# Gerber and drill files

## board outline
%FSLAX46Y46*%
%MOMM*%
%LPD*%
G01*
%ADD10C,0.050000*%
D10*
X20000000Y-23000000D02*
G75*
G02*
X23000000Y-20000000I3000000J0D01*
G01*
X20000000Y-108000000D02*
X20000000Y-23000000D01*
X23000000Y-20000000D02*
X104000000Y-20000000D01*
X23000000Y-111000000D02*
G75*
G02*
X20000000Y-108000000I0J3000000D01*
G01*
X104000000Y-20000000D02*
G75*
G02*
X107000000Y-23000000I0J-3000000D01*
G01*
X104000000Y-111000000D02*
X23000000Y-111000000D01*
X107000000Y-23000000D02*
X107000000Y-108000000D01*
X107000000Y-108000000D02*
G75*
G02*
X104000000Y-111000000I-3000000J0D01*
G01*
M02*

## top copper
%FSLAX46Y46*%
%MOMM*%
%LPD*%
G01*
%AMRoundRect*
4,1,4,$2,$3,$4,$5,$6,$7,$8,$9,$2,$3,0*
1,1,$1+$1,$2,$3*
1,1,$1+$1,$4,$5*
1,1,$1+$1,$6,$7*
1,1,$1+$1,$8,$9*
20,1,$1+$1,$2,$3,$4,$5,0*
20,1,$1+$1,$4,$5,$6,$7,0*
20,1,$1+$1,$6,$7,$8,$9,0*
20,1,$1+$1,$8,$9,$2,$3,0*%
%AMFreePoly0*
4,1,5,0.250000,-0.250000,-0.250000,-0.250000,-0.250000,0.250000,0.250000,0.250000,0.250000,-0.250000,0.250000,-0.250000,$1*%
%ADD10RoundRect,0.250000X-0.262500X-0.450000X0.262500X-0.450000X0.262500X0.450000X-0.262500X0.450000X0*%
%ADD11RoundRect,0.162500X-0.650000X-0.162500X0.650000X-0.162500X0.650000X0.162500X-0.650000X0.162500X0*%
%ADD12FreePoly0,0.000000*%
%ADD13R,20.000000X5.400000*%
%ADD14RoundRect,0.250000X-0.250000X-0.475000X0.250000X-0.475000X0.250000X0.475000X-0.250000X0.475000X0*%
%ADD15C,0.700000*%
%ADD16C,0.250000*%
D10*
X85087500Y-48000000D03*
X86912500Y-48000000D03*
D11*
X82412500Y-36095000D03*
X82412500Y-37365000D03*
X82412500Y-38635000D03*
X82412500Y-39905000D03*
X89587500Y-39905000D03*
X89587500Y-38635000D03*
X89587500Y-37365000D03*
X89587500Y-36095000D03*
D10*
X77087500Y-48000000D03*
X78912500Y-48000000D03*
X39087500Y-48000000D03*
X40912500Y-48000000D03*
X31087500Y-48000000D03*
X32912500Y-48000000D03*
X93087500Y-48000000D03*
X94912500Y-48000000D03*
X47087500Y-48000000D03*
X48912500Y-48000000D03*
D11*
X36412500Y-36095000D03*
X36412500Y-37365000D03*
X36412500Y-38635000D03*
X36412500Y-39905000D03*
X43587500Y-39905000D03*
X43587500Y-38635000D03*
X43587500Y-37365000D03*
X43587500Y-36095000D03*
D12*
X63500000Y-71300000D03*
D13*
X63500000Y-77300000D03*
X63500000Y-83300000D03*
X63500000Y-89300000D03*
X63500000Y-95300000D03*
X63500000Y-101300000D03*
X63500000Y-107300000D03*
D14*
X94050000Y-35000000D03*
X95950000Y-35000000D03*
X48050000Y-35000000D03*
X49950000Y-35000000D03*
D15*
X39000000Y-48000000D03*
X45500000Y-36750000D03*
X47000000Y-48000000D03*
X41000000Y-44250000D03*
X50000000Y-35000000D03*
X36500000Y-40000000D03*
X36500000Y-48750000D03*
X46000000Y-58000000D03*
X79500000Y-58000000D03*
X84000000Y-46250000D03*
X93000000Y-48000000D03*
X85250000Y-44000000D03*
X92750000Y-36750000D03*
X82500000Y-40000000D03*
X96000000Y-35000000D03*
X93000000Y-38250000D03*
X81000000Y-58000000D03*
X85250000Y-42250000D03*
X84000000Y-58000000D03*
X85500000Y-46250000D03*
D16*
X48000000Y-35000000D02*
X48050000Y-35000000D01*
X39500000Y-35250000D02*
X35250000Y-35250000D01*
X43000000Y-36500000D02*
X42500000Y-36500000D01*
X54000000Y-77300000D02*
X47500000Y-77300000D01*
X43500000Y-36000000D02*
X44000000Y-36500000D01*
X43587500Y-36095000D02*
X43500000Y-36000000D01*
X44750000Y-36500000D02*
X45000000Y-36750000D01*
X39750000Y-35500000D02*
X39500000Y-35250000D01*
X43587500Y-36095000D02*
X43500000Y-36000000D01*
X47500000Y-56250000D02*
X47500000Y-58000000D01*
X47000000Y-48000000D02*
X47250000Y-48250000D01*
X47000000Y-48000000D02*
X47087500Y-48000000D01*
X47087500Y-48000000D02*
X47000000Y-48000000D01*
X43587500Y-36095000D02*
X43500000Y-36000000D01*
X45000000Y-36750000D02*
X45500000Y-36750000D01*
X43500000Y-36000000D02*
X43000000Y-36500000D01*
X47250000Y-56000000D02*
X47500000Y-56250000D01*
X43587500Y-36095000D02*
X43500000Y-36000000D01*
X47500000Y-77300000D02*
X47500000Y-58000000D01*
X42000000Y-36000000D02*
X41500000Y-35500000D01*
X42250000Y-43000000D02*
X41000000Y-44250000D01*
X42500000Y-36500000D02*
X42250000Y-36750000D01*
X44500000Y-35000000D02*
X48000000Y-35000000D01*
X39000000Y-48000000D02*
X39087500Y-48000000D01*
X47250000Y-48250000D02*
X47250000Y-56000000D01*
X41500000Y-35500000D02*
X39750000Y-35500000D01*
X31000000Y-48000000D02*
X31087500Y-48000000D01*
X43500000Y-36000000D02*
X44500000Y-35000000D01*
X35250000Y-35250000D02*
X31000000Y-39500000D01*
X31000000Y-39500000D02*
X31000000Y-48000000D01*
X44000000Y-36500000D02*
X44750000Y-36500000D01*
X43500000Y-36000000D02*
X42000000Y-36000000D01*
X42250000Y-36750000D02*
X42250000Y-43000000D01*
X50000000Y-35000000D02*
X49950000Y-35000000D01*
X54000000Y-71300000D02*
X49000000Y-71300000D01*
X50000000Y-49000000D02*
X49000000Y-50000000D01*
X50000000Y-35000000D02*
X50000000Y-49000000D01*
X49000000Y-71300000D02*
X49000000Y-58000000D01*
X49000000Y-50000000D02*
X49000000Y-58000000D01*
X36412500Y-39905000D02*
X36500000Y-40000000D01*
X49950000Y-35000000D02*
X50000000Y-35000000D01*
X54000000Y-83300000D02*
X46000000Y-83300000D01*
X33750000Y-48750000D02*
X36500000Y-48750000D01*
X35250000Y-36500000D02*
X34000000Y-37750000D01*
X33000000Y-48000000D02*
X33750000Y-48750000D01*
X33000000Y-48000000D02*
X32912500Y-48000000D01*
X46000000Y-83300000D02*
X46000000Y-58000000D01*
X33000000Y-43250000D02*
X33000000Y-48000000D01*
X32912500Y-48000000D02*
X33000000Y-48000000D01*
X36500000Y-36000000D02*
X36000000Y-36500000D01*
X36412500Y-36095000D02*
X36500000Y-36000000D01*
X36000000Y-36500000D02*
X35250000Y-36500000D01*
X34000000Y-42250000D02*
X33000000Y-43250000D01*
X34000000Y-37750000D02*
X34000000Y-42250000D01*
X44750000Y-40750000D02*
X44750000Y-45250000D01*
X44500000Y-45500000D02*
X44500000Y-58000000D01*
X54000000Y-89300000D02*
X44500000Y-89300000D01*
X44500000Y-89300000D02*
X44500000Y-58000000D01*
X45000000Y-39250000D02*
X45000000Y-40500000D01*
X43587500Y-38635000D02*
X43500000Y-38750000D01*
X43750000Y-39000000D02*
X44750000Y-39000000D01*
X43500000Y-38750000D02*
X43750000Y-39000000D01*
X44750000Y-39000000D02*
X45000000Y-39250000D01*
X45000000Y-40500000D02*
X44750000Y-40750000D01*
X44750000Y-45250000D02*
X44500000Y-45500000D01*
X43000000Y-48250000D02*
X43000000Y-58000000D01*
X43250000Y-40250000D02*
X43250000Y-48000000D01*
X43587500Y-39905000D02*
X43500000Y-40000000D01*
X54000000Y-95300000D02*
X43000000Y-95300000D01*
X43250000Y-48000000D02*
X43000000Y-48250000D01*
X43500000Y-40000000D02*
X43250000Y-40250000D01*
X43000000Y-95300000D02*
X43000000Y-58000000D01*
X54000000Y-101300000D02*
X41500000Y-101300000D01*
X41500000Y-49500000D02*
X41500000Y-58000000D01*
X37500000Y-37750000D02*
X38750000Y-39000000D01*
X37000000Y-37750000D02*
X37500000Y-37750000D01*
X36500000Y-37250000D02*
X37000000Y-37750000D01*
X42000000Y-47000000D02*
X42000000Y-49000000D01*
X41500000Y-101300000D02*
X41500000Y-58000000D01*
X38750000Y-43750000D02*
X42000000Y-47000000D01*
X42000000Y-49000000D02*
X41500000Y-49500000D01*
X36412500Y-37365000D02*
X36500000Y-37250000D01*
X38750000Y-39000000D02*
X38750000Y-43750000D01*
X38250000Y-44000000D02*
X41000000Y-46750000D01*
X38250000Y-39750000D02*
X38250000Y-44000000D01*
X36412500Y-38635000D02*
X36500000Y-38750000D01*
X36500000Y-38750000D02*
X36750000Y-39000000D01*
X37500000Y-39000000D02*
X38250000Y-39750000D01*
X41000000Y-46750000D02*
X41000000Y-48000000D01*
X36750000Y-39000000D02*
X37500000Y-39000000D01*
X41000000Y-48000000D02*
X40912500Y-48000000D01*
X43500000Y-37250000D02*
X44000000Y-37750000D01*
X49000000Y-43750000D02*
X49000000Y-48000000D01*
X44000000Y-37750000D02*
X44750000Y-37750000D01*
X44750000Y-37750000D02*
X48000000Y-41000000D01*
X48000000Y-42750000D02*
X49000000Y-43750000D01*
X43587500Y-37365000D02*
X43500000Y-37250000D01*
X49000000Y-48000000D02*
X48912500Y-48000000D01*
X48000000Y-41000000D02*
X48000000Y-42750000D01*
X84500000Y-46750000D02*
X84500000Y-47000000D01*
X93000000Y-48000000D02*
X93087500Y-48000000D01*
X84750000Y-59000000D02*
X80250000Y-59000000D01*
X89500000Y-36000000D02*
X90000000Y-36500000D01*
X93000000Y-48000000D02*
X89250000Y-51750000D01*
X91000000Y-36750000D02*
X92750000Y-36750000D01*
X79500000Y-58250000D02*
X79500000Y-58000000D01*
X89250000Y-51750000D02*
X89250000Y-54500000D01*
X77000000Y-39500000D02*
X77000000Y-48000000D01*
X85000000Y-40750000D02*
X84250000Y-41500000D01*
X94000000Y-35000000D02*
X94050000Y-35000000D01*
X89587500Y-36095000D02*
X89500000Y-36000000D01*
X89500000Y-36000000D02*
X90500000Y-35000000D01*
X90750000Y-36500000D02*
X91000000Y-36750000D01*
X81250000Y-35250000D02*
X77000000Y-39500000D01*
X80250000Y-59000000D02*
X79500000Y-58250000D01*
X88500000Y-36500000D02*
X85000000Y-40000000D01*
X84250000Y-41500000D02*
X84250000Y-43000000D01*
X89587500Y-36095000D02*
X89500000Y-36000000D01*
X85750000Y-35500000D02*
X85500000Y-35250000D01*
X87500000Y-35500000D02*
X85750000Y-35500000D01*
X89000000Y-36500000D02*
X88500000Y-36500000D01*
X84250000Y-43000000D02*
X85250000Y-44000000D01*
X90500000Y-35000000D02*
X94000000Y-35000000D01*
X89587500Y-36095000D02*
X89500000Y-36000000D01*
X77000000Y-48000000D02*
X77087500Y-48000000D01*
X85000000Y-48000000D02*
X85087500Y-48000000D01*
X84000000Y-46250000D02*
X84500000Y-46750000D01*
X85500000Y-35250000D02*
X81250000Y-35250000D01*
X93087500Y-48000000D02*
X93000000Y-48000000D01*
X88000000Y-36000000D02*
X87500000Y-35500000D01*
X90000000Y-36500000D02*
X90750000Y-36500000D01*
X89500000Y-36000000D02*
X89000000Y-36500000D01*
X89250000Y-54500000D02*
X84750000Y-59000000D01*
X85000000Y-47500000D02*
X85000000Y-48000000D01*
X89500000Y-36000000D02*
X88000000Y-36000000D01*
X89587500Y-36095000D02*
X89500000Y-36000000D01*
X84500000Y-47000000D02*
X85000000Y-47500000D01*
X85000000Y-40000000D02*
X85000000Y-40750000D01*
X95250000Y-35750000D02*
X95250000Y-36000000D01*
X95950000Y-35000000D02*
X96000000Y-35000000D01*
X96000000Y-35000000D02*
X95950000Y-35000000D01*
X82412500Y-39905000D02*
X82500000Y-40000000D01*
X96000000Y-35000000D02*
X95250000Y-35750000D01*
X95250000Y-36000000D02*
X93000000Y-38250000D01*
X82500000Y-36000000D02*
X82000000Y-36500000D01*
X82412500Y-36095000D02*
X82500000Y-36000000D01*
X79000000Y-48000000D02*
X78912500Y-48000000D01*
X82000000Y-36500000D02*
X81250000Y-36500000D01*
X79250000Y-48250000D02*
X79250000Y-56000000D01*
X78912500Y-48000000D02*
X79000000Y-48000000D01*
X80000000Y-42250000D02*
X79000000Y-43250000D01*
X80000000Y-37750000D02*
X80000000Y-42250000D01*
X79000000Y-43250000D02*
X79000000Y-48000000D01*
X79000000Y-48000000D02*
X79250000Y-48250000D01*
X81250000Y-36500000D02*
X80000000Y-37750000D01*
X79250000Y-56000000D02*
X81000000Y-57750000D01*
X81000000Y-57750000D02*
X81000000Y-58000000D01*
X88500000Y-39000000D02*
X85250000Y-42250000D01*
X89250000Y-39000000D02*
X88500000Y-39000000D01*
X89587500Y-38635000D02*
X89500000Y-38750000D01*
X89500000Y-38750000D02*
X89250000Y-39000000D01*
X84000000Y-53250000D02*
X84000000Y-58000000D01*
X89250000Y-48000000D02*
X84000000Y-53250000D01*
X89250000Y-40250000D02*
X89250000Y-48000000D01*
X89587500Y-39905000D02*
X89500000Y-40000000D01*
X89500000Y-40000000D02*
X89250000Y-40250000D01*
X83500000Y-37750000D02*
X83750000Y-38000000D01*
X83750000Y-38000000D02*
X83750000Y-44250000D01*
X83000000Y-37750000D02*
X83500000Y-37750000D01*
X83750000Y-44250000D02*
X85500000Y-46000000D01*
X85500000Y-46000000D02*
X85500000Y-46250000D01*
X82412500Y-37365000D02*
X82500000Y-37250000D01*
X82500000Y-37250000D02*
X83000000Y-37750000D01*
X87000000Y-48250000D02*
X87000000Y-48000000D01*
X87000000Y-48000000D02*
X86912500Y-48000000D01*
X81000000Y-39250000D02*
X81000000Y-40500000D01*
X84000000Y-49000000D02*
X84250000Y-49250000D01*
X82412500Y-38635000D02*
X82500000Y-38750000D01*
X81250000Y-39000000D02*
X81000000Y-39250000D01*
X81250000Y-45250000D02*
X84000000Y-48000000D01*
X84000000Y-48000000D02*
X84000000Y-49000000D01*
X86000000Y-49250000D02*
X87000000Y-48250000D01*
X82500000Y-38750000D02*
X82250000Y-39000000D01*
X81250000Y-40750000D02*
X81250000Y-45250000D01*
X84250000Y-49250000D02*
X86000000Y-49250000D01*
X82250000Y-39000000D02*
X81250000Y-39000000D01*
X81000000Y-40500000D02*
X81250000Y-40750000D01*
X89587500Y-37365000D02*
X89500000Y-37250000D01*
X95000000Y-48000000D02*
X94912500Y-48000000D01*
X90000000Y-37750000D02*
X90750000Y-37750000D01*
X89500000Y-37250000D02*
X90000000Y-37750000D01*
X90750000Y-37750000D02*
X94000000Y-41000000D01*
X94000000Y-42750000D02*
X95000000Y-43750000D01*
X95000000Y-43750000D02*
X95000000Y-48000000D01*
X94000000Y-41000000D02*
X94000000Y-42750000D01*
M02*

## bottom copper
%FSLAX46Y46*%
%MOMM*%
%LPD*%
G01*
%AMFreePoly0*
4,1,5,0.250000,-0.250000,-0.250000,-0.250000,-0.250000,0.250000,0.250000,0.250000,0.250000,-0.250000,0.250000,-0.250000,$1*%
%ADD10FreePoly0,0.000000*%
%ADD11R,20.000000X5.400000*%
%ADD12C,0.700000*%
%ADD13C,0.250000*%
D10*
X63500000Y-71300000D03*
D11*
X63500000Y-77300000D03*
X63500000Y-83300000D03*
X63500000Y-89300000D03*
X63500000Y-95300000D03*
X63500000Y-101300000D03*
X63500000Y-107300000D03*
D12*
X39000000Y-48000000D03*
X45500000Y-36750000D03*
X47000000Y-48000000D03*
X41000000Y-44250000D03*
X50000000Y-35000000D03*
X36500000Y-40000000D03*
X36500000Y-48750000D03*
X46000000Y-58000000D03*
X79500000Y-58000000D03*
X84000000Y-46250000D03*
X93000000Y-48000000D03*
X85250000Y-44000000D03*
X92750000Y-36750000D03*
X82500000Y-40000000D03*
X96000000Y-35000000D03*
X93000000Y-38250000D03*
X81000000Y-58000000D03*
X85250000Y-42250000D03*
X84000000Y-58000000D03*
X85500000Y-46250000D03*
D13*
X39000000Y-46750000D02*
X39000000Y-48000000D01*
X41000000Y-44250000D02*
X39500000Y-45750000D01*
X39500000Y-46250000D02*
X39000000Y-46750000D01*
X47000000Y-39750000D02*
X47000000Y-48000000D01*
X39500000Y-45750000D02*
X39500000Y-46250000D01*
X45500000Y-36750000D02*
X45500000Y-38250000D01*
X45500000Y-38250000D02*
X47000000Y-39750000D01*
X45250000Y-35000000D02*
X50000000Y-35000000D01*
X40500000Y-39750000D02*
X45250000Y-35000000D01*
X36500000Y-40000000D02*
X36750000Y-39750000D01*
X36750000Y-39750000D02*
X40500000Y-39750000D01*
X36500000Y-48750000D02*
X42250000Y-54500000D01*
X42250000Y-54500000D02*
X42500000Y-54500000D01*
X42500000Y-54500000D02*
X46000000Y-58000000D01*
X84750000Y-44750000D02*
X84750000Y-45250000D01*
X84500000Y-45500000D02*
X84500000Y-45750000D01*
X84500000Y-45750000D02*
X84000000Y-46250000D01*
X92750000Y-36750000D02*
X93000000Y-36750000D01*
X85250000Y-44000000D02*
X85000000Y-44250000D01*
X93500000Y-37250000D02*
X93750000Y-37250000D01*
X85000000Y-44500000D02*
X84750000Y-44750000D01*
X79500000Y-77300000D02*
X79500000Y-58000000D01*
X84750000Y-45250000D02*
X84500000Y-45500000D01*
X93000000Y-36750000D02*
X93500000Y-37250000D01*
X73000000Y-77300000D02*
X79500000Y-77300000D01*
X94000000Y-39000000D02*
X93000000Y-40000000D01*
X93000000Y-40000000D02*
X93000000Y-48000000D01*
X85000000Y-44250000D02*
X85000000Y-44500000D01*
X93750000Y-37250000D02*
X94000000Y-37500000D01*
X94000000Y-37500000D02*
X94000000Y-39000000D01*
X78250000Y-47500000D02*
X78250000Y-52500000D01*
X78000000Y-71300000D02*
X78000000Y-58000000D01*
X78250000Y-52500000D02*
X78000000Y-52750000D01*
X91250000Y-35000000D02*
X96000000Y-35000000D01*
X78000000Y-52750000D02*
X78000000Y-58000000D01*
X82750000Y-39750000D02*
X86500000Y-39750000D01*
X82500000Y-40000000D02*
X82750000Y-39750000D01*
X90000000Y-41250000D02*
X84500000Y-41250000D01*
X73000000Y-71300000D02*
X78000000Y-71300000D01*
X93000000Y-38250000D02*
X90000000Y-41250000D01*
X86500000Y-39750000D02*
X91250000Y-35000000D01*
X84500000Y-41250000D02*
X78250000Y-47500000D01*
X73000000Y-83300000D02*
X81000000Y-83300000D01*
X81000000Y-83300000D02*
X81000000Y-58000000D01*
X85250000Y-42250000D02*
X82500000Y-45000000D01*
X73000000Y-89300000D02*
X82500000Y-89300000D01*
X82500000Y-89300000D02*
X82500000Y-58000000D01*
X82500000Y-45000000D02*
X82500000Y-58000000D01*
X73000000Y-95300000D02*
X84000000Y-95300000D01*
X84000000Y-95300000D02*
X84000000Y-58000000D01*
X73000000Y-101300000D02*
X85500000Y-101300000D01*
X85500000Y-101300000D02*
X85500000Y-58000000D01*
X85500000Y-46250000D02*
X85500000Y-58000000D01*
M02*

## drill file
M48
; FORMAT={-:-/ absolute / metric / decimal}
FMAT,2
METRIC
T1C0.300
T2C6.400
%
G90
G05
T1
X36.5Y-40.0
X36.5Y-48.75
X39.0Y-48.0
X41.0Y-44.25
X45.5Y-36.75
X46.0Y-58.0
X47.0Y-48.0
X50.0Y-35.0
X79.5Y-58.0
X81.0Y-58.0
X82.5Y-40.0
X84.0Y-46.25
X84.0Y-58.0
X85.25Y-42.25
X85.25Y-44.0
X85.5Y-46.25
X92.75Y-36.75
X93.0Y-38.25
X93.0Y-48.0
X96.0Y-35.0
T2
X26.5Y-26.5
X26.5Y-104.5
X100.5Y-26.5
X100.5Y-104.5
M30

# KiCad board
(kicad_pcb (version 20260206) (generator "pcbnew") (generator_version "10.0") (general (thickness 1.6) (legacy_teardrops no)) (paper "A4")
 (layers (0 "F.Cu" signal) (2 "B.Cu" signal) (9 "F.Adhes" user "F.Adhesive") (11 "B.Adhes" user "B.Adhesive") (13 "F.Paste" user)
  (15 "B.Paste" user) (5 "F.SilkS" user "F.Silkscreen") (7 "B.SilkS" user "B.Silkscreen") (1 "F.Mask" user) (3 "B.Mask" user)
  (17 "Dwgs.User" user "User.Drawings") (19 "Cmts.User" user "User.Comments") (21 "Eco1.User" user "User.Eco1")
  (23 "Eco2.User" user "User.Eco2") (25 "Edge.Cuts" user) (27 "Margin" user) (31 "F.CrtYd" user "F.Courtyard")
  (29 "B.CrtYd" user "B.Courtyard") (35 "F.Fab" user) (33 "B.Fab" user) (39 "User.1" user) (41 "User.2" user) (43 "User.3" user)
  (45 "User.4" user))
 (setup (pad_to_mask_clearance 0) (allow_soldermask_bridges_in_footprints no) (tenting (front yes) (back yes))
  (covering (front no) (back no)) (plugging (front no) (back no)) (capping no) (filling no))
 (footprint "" (layer "F.Cu") (at 100.5 104.5)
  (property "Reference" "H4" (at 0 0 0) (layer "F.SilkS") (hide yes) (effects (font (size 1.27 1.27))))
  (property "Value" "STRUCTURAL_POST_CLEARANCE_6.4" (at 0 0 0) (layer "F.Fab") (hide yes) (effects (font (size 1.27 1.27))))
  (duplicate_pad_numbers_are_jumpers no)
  (pad "" np_thru_hole circle (at 0 0) (size 6.4 6.4) (drill 6.4) (layers "*.Cu")))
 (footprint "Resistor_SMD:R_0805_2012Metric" (layer "F.Cu") (at 86 48)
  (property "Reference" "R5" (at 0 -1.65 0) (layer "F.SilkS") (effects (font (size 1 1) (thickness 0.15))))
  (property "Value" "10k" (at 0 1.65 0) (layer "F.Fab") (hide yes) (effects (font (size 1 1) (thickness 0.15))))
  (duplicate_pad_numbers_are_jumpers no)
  (pad "1" smd roundrect (at -0.9125 0) (size 1.025 1.4) (layers "F.Cu" "F.Mask" "F.Paste") (roundrect_rratio 0.243902) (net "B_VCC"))
  (pad "2" smd roundrect (at 0.9125 0) (size 1.025 1.4) (layers "F.Cu" "F.Mask" "F.Paste") (roundrect_rratio 0.243902) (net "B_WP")))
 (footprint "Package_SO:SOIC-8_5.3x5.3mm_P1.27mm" (layer "F.Cu") (at 86 38)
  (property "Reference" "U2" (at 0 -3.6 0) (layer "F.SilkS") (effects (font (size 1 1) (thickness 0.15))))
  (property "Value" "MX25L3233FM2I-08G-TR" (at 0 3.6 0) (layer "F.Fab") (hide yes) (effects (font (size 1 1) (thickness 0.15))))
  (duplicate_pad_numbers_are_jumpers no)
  (pad "1" smd roundrect (at -3.5875 -1.905) (size 1.625 0.65) (layers "F.Cu" "F.Mask" "F.Paste") (roundrect_rratio 0.25) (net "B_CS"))
  (pad "2" smd roundrect (at -3.5875 -0.635) (size 1.625 0.65) (layers "F.Cu" "F.Mask" "F.Paste") (roundrect_rratio 0.25) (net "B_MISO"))
  (pad "3" smd roundrect (at -3.5875 0.635) (size 1.625 0.65) (layers "F.Cu" "F.Mask" "F.Paste") (roundrect_rratio 0.25) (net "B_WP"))
  (pad "4" smd roundrect (at -3.5875 1.905) (size 1.625 0.65) (layers "F.Cu" "F.Mask" "F.Paste") (roundrect_rratio 0.25) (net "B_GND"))
  (pad "5" smd roundrect (at 3.5875 1.905) (size 1.625 0.65) (layers "F.Cu" "F.Mask" "F.Paste") (roundrect_rratio 0.25) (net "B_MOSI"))
  (pad "6" smd roundrect (at 3.5875 0.635) (size 1.625 0.65) (layers "F.Cu" "F.Mask" "F.Paste") (roundrect_rratio 0.25) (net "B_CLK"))
  (pad "7" smd roundrect (at 3.5875 -0.635) (size 1.625 0.65) (layers "F.Cu" "F.Mask" "F.Paste") (roundrect_rratio 0.25) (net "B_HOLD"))
  (pad "8" smd roundrect (at 3.5875 -1.905) (size 1.625 0.65) (layers "F.Cu" "F.Mask" "F.Paste") (roundrect_rratio 0.25) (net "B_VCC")))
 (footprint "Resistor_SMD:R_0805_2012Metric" (layer "F.Cu") (at 78 48)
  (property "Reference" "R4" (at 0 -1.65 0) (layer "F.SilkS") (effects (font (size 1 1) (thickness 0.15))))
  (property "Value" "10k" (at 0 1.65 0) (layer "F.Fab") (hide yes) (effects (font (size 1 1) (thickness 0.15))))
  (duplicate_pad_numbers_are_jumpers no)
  (pad "1" smd roundrect (at -0.9125 0) (size 1.025 1.4) (layers "F.Cu" "F.Mask" "F.Paste") (roundrect_rratio 0.243902) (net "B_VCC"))
  (pad "2" smd roundrect (at 0.9125 0) (size 1.025 1.4) (layers "F.Cu" "F.Mask" "F.Paste") (roundrect_rratio 0.243902) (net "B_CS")))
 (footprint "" (layer "F.Cu") (at 100.5 26.5)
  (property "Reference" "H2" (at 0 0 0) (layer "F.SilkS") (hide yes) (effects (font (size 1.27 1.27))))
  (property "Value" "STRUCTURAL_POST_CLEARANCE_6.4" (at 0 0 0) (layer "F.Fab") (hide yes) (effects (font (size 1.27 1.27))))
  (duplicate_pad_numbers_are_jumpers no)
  (pad "" np_thru_hole circle (at 0 0) (size 6.4 6.4) (drill 6.4) (layers "*.Cu")))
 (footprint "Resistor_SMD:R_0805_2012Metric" (layer "F.Cu") (at 40 48)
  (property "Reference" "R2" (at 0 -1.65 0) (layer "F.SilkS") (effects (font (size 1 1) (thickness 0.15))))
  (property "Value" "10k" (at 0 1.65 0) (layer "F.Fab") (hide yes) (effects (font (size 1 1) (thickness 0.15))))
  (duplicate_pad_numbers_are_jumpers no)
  (pad "1" smd roundrect (at -0.9125 0) (size 1.025 1.4) (layers "F.Cu" "F.Mask" "F.Paste") (roundrect_rratio 0.243902) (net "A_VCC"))
  (pad "2" smd roundrect (at 0.9125 0) (size 1.025 1.4) (layers "F.Cu" "F.Mask" "F.Paste") (roundrect_rratio 0.243902) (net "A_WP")))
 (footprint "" (layer "F.Cu") (at 26.5 26.5)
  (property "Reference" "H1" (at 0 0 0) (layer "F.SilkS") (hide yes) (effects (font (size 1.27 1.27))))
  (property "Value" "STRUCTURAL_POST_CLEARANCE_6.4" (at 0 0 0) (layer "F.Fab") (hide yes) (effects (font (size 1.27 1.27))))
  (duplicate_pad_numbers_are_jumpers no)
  (pad "" np_thru_hole circle (at 0 0) (size 6.4 6.4) (drill 6.4) (layers "*.Cu")))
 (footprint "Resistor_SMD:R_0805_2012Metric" (layer "F.Cu") (at 32 48)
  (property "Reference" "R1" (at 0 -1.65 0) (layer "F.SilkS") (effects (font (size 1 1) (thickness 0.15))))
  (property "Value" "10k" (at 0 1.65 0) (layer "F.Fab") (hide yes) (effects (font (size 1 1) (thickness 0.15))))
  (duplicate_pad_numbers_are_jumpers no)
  (pad "1" smd roundrect (at -0.9125 0) (size 1.025 1.4) (layers "F.Cu" "F.Mask" "F.Paste") (roundrect_rratio 0.243902) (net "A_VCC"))
  (pad "2" smd roundrect (at 0.9125 0) (size 1.025 1.4) (layers "F.Cu" "F.Mask" "F.Paste") (roundrect_rratio 0.243902) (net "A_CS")))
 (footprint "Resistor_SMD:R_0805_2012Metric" (layer "F.Cu") (at 94 48)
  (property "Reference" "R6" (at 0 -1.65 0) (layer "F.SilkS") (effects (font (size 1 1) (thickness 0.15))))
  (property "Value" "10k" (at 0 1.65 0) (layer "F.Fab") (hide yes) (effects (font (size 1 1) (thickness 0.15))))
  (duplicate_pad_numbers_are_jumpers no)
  (pad "1" smd roundrect (at -0.9125 0) (size 1.025 1.4) (layers "F.Cu" "F.Mask" "F.Paste") (roundrect_rratio 0.243902) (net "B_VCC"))
  (pad "2" smd roundrect (at 0.9125 0) (size 1.025 1.4) (layers "F.Cu" "F.Mask" "F.Paste") (roundrect_rratio 0.243902) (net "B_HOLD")))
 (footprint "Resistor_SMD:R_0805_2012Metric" (layer "F.Cu") (at 48 48)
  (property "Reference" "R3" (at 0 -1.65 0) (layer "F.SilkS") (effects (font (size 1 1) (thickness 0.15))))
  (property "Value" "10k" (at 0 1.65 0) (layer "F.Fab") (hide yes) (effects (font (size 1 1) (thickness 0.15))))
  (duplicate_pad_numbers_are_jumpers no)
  (pad "1" smd roundrect (at -0.9125 0) (size 1.025 1.4) (layers "F.Cu" "F.Mask" "F.Paste") (roundrect_rratio 0.243902) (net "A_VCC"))
  (pad "2" smd roundrect (at 0.9125 0) (size 1.025 1.4) (layers "F.Cu" "F.Mask" "F.Paste") (roundrect_rratio 0.243902) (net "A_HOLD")))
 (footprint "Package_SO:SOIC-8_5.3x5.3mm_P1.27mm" (layer "F.Cu") (at 40 38)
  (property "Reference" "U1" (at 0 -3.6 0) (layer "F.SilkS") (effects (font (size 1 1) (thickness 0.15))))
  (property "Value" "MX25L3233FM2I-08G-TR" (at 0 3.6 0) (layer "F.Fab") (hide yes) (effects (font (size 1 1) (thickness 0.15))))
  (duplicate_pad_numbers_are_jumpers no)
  (pad "1" smd roundrect (at -3.5875 -1.905) (size 1.625 0.65) (layers "F.Cu" "F.Mask" "F.Paste") (roundrect_rratio 0.25) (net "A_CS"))
  (pad "2" smd roundrect (at -3.5875 -0.635) (size 1.625 0.65) (layers "F.Cu" "F.Mask" "F.Paste") (roundrect_rratio 0.25) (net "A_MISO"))
  (pad "3" smd roundrect (at -3.5875 0.635) (size 1.625 0.65) (layers "F.Cu" "F.Mask" "F.Paste") (roundrect_rratio 0.25) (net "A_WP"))
  (pad "4" smd roundrect (at -3.5875 1.905) (size 1.625 0.65) (layers "F.Cu" "F.Mask" "F.Paste") (roundrect_rratio 0.25) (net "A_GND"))
  (pad "5" smd roundrect (at 3.5875 1.905) (size 1.625 0.65) (layers "F.Cu" "F.Mask" "F.Paste") (roundrect_rratio 0.25) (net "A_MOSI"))
  (pad "6" smd roundrect (at 3.5875 0.635) (size 1.625 0.65) (layers "F.Cu" "F.Mask" "F.Paste") (roundrect_rratio 0.25) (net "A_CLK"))
  (pad "7" smd roundrect (at 3.5875 -0.635) (size 1.625 0.65) (layers "F.Cu" "F.Mask" "F.Paste") (roundrect_rratio 0.25) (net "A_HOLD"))
  (pad "8" smd roundrect (at 3.5875 -1.905) (size 1.625 0.65) (layers "F.Cu" "F.Mask" "F.Paste") (roundrect_rratio 0.25) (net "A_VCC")))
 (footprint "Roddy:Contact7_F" (layer "F.Cu") (at 63.5 0)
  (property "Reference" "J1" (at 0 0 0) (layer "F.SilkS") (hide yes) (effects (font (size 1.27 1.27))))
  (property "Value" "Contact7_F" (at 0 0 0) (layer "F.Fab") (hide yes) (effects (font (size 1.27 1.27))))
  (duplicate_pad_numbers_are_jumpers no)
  (pad "1" smd custom (at 0 71.3) (size 0.5 0.5) (layers "F.Cu" "F.Mask") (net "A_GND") (solder_mask_margin 0.05) (thermal_bridge_angle 45)
   (options (clearance outline) (anchor rect)) (primitives))
  (pad "2" smd rect (at 0 77.3) (size 20 5.4) (layers "F.Cu" "F.Mask") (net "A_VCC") (solder_mask_margin 0.05) (thermal_bridge_angle 45))
  (pad "3" smd rect (at 0 83.3) (size 20 5.4) (layers "F.Cu" "F.Mask") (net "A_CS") (solder_mask_margin 0.05) (thermal_bridge_angle 45))
  (pad "4" smd rect (at 0 89.3) (size 20 5.4) (layers "F.Cu" "F.Mask") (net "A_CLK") (solder_mask_margin 0.05) (thermal_bridge_angle 45))
  (pad "5" smd rect (at 0 95.3) (size 20 5.4) (layers "F.Cu" "F.Mask") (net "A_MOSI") (solder_mask_margin 0.05) (thermal_bridge_angle 45))
  (pad "6" smd rect (at 0 101.3) (size 20 5.4) (layers "F.Cu" "F.Mask") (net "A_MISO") (solder_mask_margin 0.05) (thermal_bridge_angle 45))
  (pad "7" smd rect (at 0 107.3) (size 20 5.4) (layers "F.Cu" "F.Mask") (solder_mask_margin 0.05) (thermal_bridge_angle 45)))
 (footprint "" (layer "F.Cu") (at 26.5 104.5)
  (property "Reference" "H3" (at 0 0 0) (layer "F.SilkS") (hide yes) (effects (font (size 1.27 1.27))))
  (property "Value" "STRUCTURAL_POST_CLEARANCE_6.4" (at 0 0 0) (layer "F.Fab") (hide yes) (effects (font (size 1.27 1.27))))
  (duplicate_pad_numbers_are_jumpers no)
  (pad "" np_thru_hole circle (at 0 0) (size 6.4 6.4) (drill 6.4) (layers "*.Cu")))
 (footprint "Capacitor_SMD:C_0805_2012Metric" (layer "F.Cu") (at 95 35)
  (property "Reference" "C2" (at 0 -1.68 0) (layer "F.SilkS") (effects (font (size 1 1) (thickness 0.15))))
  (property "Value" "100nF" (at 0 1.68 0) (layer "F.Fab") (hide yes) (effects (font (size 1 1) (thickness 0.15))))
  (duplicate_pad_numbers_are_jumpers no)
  (pad "1" smd roundrect (at -0.95 0) (size 1 1.45) (layers "F.Cu" "F.Mask" "F.Paste") (roundrect_rratio 0.25) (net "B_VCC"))
  (pad "2" smd roundrect (at 0.95 0) (size 1 1.45) (layers "F.Cu" "F.Mask" "F.Paste") (roundrect_rratio 0.25) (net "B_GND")))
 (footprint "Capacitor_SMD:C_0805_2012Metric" (layer "F.Cu") (at 49 35)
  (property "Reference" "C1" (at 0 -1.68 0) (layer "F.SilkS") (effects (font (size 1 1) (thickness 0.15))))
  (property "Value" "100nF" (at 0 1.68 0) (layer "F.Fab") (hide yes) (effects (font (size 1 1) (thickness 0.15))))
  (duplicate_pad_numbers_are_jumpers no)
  (pad "1" smd roundrect (at -0.95 0) (size 1 1.45) (layers "F.Cu" "F.Mask" "F.Paste") (roundrect_rratio 0.25) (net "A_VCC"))
  (pad "2" smd roundrect (at 0.95 0) (size 1 1.45) (layers "F.Cu" "F.Mask" "F.Paste") (roundrect_rratio 0.25) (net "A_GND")))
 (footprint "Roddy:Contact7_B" (layer "B.Cu") (at 63.5 0)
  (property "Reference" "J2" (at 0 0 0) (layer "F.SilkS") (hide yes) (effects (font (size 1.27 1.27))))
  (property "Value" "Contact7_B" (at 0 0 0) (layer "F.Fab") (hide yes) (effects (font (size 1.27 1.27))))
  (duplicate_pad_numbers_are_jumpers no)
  (pad "1" smd custom (at 0 71.3) (size 0.5 0.5) (layers "B.Cu" "B.Mask") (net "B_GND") (solder_mask_margin 0.05) (thermal_bridge_angle 45)
   (options (clearance outline) (anchor rect)) (primitives))
  (pad "2" smd rect (at 0 77.3) (size 20 5.4) (layers "B.Cu" "B.Mask") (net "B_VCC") (solder_mask_margin 0.05) (thermal_bridge_angle 45))
  (pad "3" smd rect (at 0 83.3) (size 20 5.4) (layers "B.Cu" "B.Mask") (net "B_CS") (solder_mask_margin 0.05) (thermal_bridge_angle 45))
  (pad "4" smd rect (at 0 89.3) (size 20 5.4) (layers "B.Cu" "B.Mask") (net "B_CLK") (solder_mask_margin 0.05) (thermal_bridge_angle 45))
  (pad "5" smd rect (at 0 95.3) (size 20 5.4) (layers "B.Cu" "B.Mask") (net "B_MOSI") (solder_mask_margin 0.05) (thermal_bridge_angle 45))
  (pad "6" smd rect (at 0 101.3) (size 20 5.4) (layers "B.Cu" "B.Mask") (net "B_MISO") (solder_mask_margin 0.05) (thermal_bridge_angle 45))
  (pad "7" smd rect (at 0 107.3) (size 20 5.4) (layers "B.Cu" "B.Mask") (solder_mask_margin 0.05) (thermal_bridge_angle 45)))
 (gr_arc (start 20 23) (mid 20.878679 20.878679) (end 23 20) (stroke (width 0.05) (type default)) (layer "Edge.Cuts"))
 (gr_line (start 20 108) (end 20 23) (stroke (width 0.05) (type default)) (layer "Edge.Cuts"))
 (gr_line (start 23 20) (end 104 20) (stroke (width 0.05) (type default)) (layer "Edge.Cuts"))
 (gr_arc (start 23 111) (mid 20.878679 110.12132) (end 20 108) (stroke (width 0.05) (type default)) (layer "Edge.Cuts"))
 (gr_arc (start 104 20) (mid 106.12132 20.878679) (end 107 23) (stroke (width 0.05) (type default)) (layer "Edge.Cuts"))
 (gr_line (start 104 111) (end 23 111) (stroke (width 0.05) (type default)) (layer "Edge.Cuts"))
 (gr_line (start 107 23) (end 107 108) (stroke (width 0.05) (type default)) (layer "Edge.Cuts"))
 (gr_arc (start 107 108) (mid 106.12132 110.12132) (end 104 111) (stroke (width 0.05) (type default)) (layer "Edge.Cuts"))
 (segment (start 48 35) (end 48.05 35) (width 0.25) (layer "F.Cu") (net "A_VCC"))
 (segment (start 39.5 35.25) (end 35.25 35.25) (width 0.25) (layer "F.Cu") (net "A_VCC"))
 (segment (start 43 36.5) (end 42.5 36.5) (width 0.25) (layer "F.Cu") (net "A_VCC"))
 (segment (start 54 77.3) (end 47.5 77.3) (width 0.25) (layer "F.Cu") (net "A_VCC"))
 (segment (start 43.5 36) (end 44 36.5) (width 0.25) (layer "F.Cu") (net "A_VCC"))
 (segment (start 43.5875 36.095) (end 43.5 36) (width 0.25) (layer "F.Cu") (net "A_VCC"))
 (segment (start 44.75 36.5) (end 45 36.75) (width 0.25) (layer "F.Cu") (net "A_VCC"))
 (segment (start 39.75 35.5) (end 39.5 35.25) (width 0.25) (layer "F.Cu") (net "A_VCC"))
 (segment (start 43.5875 36.095) (end 43.5 36) (width 0.25) (layer "F.Cu") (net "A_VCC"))
 (segment (start 47.5 56.25) (end 47.5 58) (width 0.25) (layer "F.Cu") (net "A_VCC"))
 (segment (start 47 48) (end 47.25 48.25) (width 0.25) (layer "F.Cu") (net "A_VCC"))
 (segment (start 47 48) (end 47.0875 48) (width 0.25) (layer "F.Cu") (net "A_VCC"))
 (segment (start 47.0875 48) (end 47 48) (width 0.25) (layer "F.Cu") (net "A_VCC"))
 (segment (start 43.5875 36.095) (end 43.5 36) (width 0.25) (layer "F.Cu") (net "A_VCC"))
 (segment (start 45 36.75) (end 45.5 36.75) (width 0.25) (layer "F.Cu") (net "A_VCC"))
 (segment (start 43.5 36) (end 43 36.5) (width 0.25) (layer "F.Cu") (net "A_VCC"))
 (segment (start 47.25 56) (end 47.5 56.25) (width 0.25) (layer "F.Cu") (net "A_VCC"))
 (segment (start 43.5875 36.095) (end 43.5 36) (width 0.25) (layer "F.Cu") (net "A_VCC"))
 (segment (start 47.5 77.3) (end 47.5 58) (width 0.25) (layer "F.Cu") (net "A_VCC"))
 (segment (start 42 36) (end 41.5 35.5) (width 0.25) (layer "F.Cu") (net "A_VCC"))
 (segment (start 42.25 43) (end 41 44.25) (width 0.25) (layer "F.Cu") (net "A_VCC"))
 (segment (start 42.5 36.5) (end 42.25 36.75) (width 0.25) (layer "F.Cu") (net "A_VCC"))
 (segment (start 44.5 35) (end 48 35) (width 0.25) (layer "F.Cu") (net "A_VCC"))
 (segment (start 39 48) (end 39.0875 48) (width 0.25) (layer "F.Cu") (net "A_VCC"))
 (segment (start 47.25 48.25) (end 47.25 56) (width 0.25) (layer "F.Cu") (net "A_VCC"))
 (segment (start 41.5 35.5) (end 39.75 35.5) (width 0.25) (layer "F.Cu") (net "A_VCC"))
 (segment (start 31 48) (end 31.0875 48) (width 0.25) (layer "F.Cu") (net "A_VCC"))
 (segment (start 43.5 36) (end 44.5 35) (width 0.25) (layer "F.Cu") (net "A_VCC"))
 (segment (start 35.25 35.25) (end 31 39.5) (width 0.25) (layer "F.Cu") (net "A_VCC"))
 (segment (start 31 39.5) (end 31 48) (width 0.25) (layer "F.Cu") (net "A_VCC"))
 (segment (start 44 36.5) (end 44.75 36.5) (width 0.25) (layer "F.Cu") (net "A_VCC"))
 (segment (start 43.5 36) (end 42 36) (width 0.25) (layer "F.Cu") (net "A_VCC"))
 (segment (start 42.25 36.75) (end 42.25 43) (width 0.25) (layer "F.Cu") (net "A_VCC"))
 (via (at 39 48) (size 0.7) (drill 0.3) (layers "F.Cu" "B.Cu") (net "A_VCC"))
 (via (at 45.5 36.75) (size 0.7) (drill 0.3) (layers "F.Cu" "B.Cu") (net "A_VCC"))
 (via (at 47 48) (size 0.7) (drill 0.3) (layers "F.Cu" "B.Cu") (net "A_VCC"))
 (via (at 41 44.25) (size 0.7) (drill 0.3) (layers "F.Cu" "B.Cu") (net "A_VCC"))
 (segment (start 39 46.75) (end 39 48) (width 0.25) (layer "B.Cu") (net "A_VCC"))
 (segment (start 41 44.25) (end 39.5 45.75) (width 0.25) (layer "B.Cu") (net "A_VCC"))
 (segment (start 39.5 46.25) (end 39 46.75) (width 0.25) (layer "B.Cu") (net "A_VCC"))
 (segment (start 47 39.75) (end 47 48) (width 0.25) (layer "B.Cu") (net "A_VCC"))
 (segment (start 39.5 45.75) (end 39.5 46.25) (width 0.25) (layer "B.Cu") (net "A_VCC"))
 (segment (start 45.5 36.75) (end 45.5 38.25) (width 0.25) (layer "B.Cu") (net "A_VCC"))
 (segment (start 45.5 38.25) (end 47 39.75) (width 0.25) (layer "B.Cu") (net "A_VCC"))
 (segment (start 50 35) (end 49.95 35) (width 0.25) (layer "F.Cu") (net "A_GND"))
 (segment (start 54 71.3) (end 49 71.3) (width 0.25) (layer "F.Cu") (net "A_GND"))
 (segment (start 50 49) (end 49 50) (width 0.25) (layer "F.Cu") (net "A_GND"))
 (segment (start 50 35) (end 50 49) (width 0.25) (layer "F.Cu") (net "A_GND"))
 (segment (start 49 71.3) (end 49 58) (width 0.25) (layer "F.Cu") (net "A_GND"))
 (segment (start 49 50) (end 49 58) (width 0.25) (layer "F.Cu") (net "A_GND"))
 (segment (start 36.4125 39.905) (end 36.5 40) (width 0.25) (layer "F.Cu") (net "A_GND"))
 (segment (start 49.95 35) (end 50 35) (width 0.25) (layer "F.Cu") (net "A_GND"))
 (via (at 50 35) (size 0.7) (drill 0.3) (layers "F.Cu" "B.Cu") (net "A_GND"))
 (via (at 36.5 40) (size 0.7) (drill 0.3) (layers "F.Cu" "B.Cu") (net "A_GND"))
 (segment (start 45.25 35) (end 50 35) (width 0.25) (layer "B.Cu") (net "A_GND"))
 (segment (start 40.5 39.75) (end 45.25 35) (width 0.25) (layer "B.Cu") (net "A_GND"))
 (segment (start 36.5 40) (end 36.75 39.75) (width 0.25) (layer "B.Cu") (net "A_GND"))
 (segment (start 36.75 39.75) (end 40.5 39.75) (width 0.25) (layer "B.Cu") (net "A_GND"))
 (segment (start 54 83.3) (end 46 83.3) (width 0.25) (layer "F.Cu") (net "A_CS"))
 (segment (start 33.75 48.75) (end 36.5 48.75) (width 0.25) (layer "F.Cu") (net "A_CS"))
 (segment (start 35.25 36.5) (end 34 37.75) (width 0.25) (layer "F.Cu") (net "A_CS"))
 (segment (start 33 48) (end 33.75 48.75) (width 0.25) (layer "F.Cu") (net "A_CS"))
 (segment (start 33 48) (end 32.9125 48) (width 0.25) (layer "F.Cu") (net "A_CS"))
 (segment (start 46 83.3) (end 46 58) (width 0.25) (layer "F.Cu") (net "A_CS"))
 (segment (start 33 43.25) (end 33 48) (width 0.25) (layer "F.Cu") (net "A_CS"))
 (segment (start 32.9125 48) (end 33 48) (width 0.25) (layer "F.Cu") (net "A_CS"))
 (segment (start 36.5 36) (end 36 36.5) (width 0.25) (layer "F.Cu") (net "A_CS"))
 (segment (start 36.4125 36.095) (end 36.5 36) (width 0.25) (layer "F.Cu") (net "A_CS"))
 (segment (start 36 36.5) (end 35.25 36.5) (width 0.25) (layer "F.Cu") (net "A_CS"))
 (segment (start 34 42.25) (end 33 43.25) (width 0.25) (layer "F.Cu") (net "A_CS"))
 (segment (start 34 37.75) (end 34 42.25) (width 0.25) (layer "F.Cu") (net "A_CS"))
 (via (at 36.5 48.75) (size 0.7) (drill 0.3) (layers "F.Cu" "B.Cu") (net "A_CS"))
 (via (at 46 58) (size 0.7) (drill 0.3) (layers "F.Cu" "B.Cu") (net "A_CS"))
 (segment (start 36.5 48.75) (end 42.25 54.5) (width 0.25) (layer "B.Cu") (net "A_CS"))
 (segment (start 42.25 54.5) (end 42.5 54.5) (width 0.25) (layer "B.Cu") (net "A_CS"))
 (segment (start 42.5 54.5) (end 46 58) (width 0.25) (layer "B.Cu") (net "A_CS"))
 (segment (start 44.75 40.75) (end 44.75 45.25) (width 0.25) (layer "F.Cu") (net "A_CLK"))
 (segment (start 44.5 45.5) (end 44.5 58) (width 0.25) (layer "F.Cu") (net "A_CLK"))
 (segment (start 54 89.3) (end 44.5 89.3) (width 0.25) (layer "F.Cu") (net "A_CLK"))
 (segment (start 44.5 89.3) (end 44.5 58) (width 0.25) (layer "F.Cu") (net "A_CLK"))
 (segment (start 45 39.25) (end 45 40.5) (width 0.25) (layer "F.Cu") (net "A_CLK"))
 (segment (start 43.5875 38.635) (end 43.5 38.75) (width 0.25) (layer "F.Cu") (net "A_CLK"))
 (segment (start 43.75 39) (end 44.75 39) (width 0.25) (layer "F.Cu") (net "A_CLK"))
 (segment (start 43.5 38.75) (end 43.75 39) (width 0.25) (layer "F.Cu") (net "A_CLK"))
 (segment (start 44.75 39) (end 45 39.25) (width 0.25) (layer "F.Cu") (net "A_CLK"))
 (segment (start 45 40.5) (end 44.75 40.75) (width 0.25) (layer "F.Cu") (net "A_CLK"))
 (segment (start 44.75 45.25) (end 44.5 45.5) (width 0.25) (layer "F.Cu") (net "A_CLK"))
 (segment (start 43 48.25) (end 43 58) (width 0.25) (layer "F.Cu") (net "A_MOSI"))
 (segment (start 43.25 40.25) (end 43.25 48) (width 0.25) (layer "F.Cu") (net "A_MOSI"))
 (segment (start 43.5875 39.905) (end 43.5 40) (width 0.25) (layer "F.Cu") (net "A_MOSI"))
 (segment (start 54 95.3) (end 43 95.3) (width 0.25) (layer "F.Cu") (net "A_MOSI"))
 (segment (start 43.25 48) (end 43 48.25) (width 0.25) (layer "F.Cu") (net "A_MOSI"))
 (segment (start 43.5 40) (end 43.25 40.25) (width 0.25) (layer "F.Cu") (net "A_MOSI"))
 (segment (start 43 95.3) (end 43 58) (width 0.25) (layer "F.Cu") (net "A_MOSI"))
 (segment (start 54 101.3) (end 41.5 101.3) (width 0.25) (layer "F.Cu") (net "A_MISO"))
 (segment (start 41.5 49.5) (end 41.5 58) (width 0.25) (layer "F.Cu") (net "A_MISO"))
 (segment (start 37.5 37.75) (end 38.75 39) (width 0.25) (layer "F.Cu") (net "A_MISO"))
 (segment (start 37 37.75) (end 37.5 37.75) (width 0.25) (layer "F.Cu") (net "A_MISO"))
 (segment (start 36.5 37.25) (end 37 37.75) (width 0.25) (layer "F.Cu") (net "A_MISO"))
 (segment (start 42 47) (end 42 49) (width 0.25) (layer "F.Cu") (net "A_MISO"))
 (segment (start 41.5 101.3) (end 41.5 58) (width 0.25) (layer "F.Cu") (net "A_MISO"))
 (segment (start 38.75 43.75) (end 42 47) (width 0.25) (layer "F.Cu") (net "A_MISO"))
 (segment (start 42 49) (end 41.5 49.5) (width 0.25) (layer "F.Cu") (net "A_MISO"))
 (segment (start 36.4125 37.365) (end 36.5 37.25) (width 0.25) (layer "F.Cu") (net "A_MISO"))
 (segment (start 38.75 39) (end 38.75 43.75) (width 0.25) (layer "F.Cu") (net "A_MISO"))
 (segment (start 38.25 44) (end 41 46.75) (width 0.25) (layer "F.Cu") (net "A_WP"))
 (segment (start 38.25 39.75) (end 38.25 44) (width 0.25) (layer "F.Cu") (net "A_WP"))
 (segment (start 36.4125 38.635) (end 36.5 38.75) (width 0.25) (layer "F.Cu") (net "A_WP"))
 (segment (start 36.5 38.75) (end 36.75 39) (width 0.25) (layer "F.Cu") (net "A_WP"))
 (segment (start 37.5 39) (end 38.25 39.75) (width 0.25) (layer "F.Cu") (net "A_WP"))
 (segment (start 41 46.75) (end 41 48) (width 0.25) (layer "F.Cu") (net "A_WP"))
 (segment (start 36.75 39) (end 37.5 39) (width 0.25) (layer "F.Cu") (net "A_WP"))
 (segment (start 41 48) (end 40.9125 48) (width 0.25) (layer "F.Cu") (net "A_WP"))
 (segment (start 43.5 37.25) (end 44 37.75) (width 0.25) (layer "F.Cu") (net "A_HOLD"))
 (segment (start 49 43.75) (end 49 48) (width 0.25) (layer "F.Cu") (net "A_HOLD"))
 (segment (start 44 37.75) (end 44.75 37.75) (width 0.25) (layer "F.Cu") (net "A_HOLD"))
 (segment (start 44.75 37.75) (end 48 41) (width 0.25) (layer "F.Cu") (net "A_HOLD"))
 (segment (start 48 42.75) (end 49 43.75) (width 0.25) (layer "F.Cu") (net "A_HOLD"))
 (segment (start 43.5875 37.365) (end 43.5 37.25) (width 0.25) (layer "F.Cu") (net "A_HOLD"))
 (segment (start 49 48) (end 48.9125 48) (width 0.25) (layer "F.Cu") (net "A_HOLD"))
 (segment (start 48 41) (end 48 42.75) (width 0.25) (layer "F.Cu") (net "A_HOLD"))
 (segment (start 84.5 46.75) (end 84.5 47) (width 0.25) (layer "F.Cu") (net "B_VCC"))
 (segment (start 93 48) (end 93.0875 48) (width 0.25) (layer "F.Cu") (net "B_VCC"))
 (segment (start 84.75 59) (end 80.25 59) (width 0.25) (layer "F.Cu") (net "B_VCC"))
 (segment (start 89.5 36) (end 90 36.5) (width 0.25) (layer "F.Cu") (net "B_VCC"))
 (segment (start 93 48) (end 89.25 51.75) (width 0.25) (layer "F.Cu") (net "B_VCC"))
 (segment (start 91 36.75) (end 92.75 36.75) (width 0.25) (layer "F.Cu") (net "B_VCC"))
 (segment (start 79.5 58.25) (end 79.5 58) (width 0.25) (layer "F.Cu") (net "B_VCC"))
 (segment (start 89.25 51.75) (end 89.25 54.5) (width 0.25) (layer "F.Cu") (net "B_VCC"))
 (segment (start 77 39.5) (end 77 48) (width 0.25) (layer "F.Cu") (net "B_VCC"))
 (segment (start 85 40.75) (end 84.25 41.5) (width 0.25) (layer "F.Cu") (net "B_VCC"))
 (segment (start 94 35) (end 94.05 35) (width 0.25) (layer "F.Cu") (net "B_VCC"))
 (segment (start 89.5875 36.095) (end 89.5 36) (width 0.25) (layer "F.Cu") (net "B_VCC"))
 (segment (start 89.5 36) (end 90.5 35) (width 0.25) (layer "F.Cu") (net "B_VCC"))
 (segment (start 90.75 36.5) (end 91 36.75) (width 0.25) (layer "F.Cu") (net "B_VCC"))
 (segment (start 81.25 35.25) (end 77 39.5) (width 0.25) (layer "F.Cu") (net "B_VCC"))
 (segment (start 80.25 59) (end 79.5 58.25) (width 0.25) (layer "F.Cu") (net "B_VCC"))
 (segment (start 88.5 36.5) (end 85 40) (width 0.25) (layer "F.Cu") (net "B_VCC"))
 (segment (start 84.25 41.5) (end 84.25 43) (width 0.25) (layer "F.Cu") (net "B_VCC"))
 (segment (start 89.5875 36.095) (end 89.5 36) (width 0.25) (layer "F.Cu") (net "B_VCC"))
 (segment (start 85.75 35.5) (end 85.5 35.25) (width 0.25) (layer "F.Cu") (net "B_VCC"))
 (segment (start 87.5 35.5) (end 85.75 35.5) (width 0.25) (layer "F.Cu") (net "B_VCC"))
 (segment (start 89 36.5) (end 88.5 36.5) (width 0.25) (layer "F.Cu") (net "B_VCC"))
 (segment (start 84.25 43) (end 85.25 44) (width 0.25) (layer "F.Cu") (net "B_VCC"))
 (segment (start 90.5 35) (end 94 35) (width 0.25) (layer "F.Cu") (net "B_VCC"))
 (segment (start 89.5875 36.095) (end 89.5 36) (width 0.25) (layer "F.Cu") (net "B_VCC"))
 (segment (start 77 48) (end 77.0875 48) (width 0.25) (layer "F.Cu") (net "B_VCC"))
 (segment (start 85 48) (end 85.0875 48) (width 0.25) (layer "F.Cu") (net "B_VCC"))
 (segment (start 84 46.25) (end 84.5 46.75) (width 0.25) (layer "F.Cu") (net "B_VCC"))
 (segment (start 85.5 35.25) (end 81.25 35.25) (width 0.25) (layer "F.Cu") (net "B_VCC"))
 (segment (start 93.0875 48) (end 93 48) (width 0.25) (layer "F.Cu") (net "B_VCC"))
 (segment (start 88 36) (end 87.5 35.5) (width 0.25) (layer "F.Cu") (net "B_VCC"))
 (segment (start 90 36.5) (end 90.75 36.5) (width 0.25) (layer "F.Cu") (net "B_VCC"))
 (segment (start 89.5 36) (end 89 36.5) (width 0.25) (layer "F.Cu") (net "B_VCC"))
 (segment (start 89.25 54.5) (end 84.75 59) (width 0.25) (layer "F.Cu") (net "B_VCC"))
 (segment (start 85 47.5) (end 85 48) (width 0.25) (layer "F.Cu") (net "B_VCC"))
 (segment (start 89.5 36) (end 88 36) (width 0.25) (layer "F.Cu") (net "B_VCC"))
 (segment (start 89.5875 36.095) (end 89.5 36) (width 0.25) (layer "F.Cu") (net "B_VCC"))
 (segment (start 84.5 47) (end 85 47.5) (width 0.25) (layer "F.Cu") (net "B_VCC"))
 (segment (start 85 40) (end 85 40.75) (width 0.25) (layer "F.Cu") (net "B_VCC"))
 (via (at 79.5 58) (size 0.7) (drill 0.3) (layers "F.Cu" "B.Cu") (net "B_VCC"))
 (via (at 84 46.25) (size 0.7) (drill 0.3) (layers "F.Cu" "B.Cu") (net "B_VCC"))
 (via (at 93 48) (size 0.7) (drill 0.3) (layers "F.Cu" "B.Cu") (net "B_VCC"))
 (via (at 85.25 44) (size 0.7) (drill 0.3) (layers "F.Cu" "B.Cu") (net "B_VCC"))
 (via (at 92.75 36.75) (size 0.7) (drill 0.3) (layers "F.Cu" "B.Cu") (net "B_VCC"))
 (segment (start 84.75 44.75) (end 84.75 45.25) (width 0.25) (layer "B.Cu") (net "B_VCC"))
 (segment (start 84.5 45.5) (end 84.5 45.75) (width 0.25) (layer "B.Cu") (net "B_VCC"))
 (segment (start 84.5 45.75) (end 84 46.25) (width 0.25) (layer "B.Cu") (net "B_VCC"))
 (segment (start 92.75 36.75) (end 93 36.75) (width 0.25) (layer "B.Cu") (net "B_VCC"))
 (segment (start 85.25 44) (end 85 44.25) (width 0.25) (layer "B.Cu") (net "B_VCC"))
 (segment (start 93.5 37.25) (end 93.75 37.25) (width 0.25) (layer "B.Cu") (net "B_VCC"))
 (segment (start 85 44.5) (end 84.75 44.75) (width 0.25) (layer "B.Cu") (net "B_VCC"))
 (segment (start 79.5 77.3) (end 79.5 58) (width 0.25) (layer "B.Cu") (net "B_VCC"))
 (segment (start 84.75 45.25) (end 84.5 45.5) (width 0.25) (layer "B.Cu") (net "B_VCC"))
 (segment (start 93 36.75) (end 93.5 37.25) (width 0.25) (layer "B.Cu") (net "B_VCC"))
 (segment (start 73 77.3) (end 79.5 77.3) (width 0.25) (layer "B.Cu") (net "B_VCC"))
 (segment (start 94 39) (end 93 40) (width 0.25) (layer "B.Cu") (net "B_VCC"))
 (segment (start 93 40) (end 93 48) (width 0.25) (layer "B.Cu") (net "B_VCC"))
 (segment (start 85 44.25) (end 85 44.5) (width 0.25) (layer "B.Cu") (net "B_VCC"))
 (segment (start 93.75 37.25) (end 94 37.5) (width 0.25) (layer "B.Cu") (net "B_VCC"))
 (segment (start 94 37.5) (end 94 39) (width 0.25) (layer "B.Cu") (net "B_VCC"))
 (segment (start 95.25 35.75) (end 95.25 36) (width 0.25) (layer "F.Cu") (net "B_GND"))
 (segment (start 95.95 35) (end 96 35) (width 0.25) (layer "F.Cu") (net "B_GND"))
 (segment (start 96 35) (end 95.95 35) (width 0.25) (layer "F.Cu") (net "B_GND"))
 (segment (start 82.4125 39.905) (end 82.5 40) (width 0.25) (layer "F.Cu") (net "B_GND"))
 (segment (start 96 35) (end 95.25 35.75) (width 0.25) (layer "F.Cu") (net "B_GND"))
 (segment (start 95.25 36) (end 93 38.25) (width 0.25) (layer "F.Cu") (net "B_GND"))
 (via (at 82.5 40) (size 0.7) (drill 0.3) (layers "F.Cu" "B.Cu") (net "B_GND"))
 (via (at 96 35) (size 0.7) (drill 0.3) (layers "F.Cu" "B.Cu") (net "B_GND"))
 (via (at 93 38.25) (size 0.7) (drill 0.3) (layers "F.Cu" "B.Cu") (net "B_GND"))
 (segment (start 78.25 47.5) (end 78.25 52.5) (width 0.25) (layer "B.Cu") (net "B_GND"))
 (segment (start 78 71.3) (end 78 58) (width 0.25) (layer "B.Cu") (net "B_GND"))
 (segment (start 78.25 52.5) (end 78 52.75) (width 0.25) (layer "B.Cu") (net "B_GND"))
 (segment (start 91.25 35) (end 96 35) (width 0.25) (layer "B.Cu") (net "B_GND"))
 (segment (start 78 52.75) (end 78 58) (width 0.25) (layer "B.Cu") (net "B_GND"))
 (segment (start 82.75 39.75) (end 86.5 39.75) (width 0.25) (layer "B.Cu") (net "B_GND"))
 (segment (start 82.5 40) (end 82.75 39.75) (width 0.25) (layer "B.Cu") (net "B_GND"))
 (segment (start 90 41.25) (end 84.5 41.25) (width 0.25) (layer "B.Cu") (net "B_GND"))
 (segment (start 73 71.3) (end 78 71.3) (width 0.25) (layer "B.Cu") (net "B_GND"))
 (segment (start 93 38.25) (end 90 41.25) (width 0.25) (layer "B.Cu") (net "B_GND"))
 (segment (start 86.5 39.75) (end 91.25 35) (width 0.25) (layer "B.Cu") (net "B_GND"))
 (segment (start 84.5 41.25) (end 78.25 47.5) (width 0.25) (layer "B.Cu") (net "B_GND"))
 (segment (start 82.5 36) (end 82 36.5) (width 0.25) (layer "F.Cu") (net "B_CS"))
 (segment (start 82.4125 36.095) (end 82.5 36) (width 0.25) (layer "F.Cu") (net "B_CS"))
 (segment (start 79 48) (end 78.9125 48) (width 0.25) (layer "F.Cu") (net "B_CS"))
 (segment (start 82 36.5) (end 81.25 36.5) (width 0.25) (layer "F.Cu") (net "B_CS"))
 (segment (start 79.25 48.25) (end 79.25 56) (width 0.25) (layer "F.Cu") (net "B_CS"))
 (segment (start 78.9125 48) (end 79 48) (width 0.25) (layer "F.Cu") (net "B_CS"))
 (segment (start 80 42.25) (end 79 43.25) (width 0.25) (layer "F.Cu") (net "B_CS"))
 (segment (start 80 37.75) (end 80 42.25) (width 0.25) (layer "F.Cu") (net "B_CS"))
 (segment (start 79 43.25) (end 79 48) (width 0.25) (layer "F.Cu") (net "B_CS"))
 (segment (start 79 48) (end 79.25 48.25) (width 0.25) (layer "F.Cu") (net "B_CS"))
 (segment (start 81.25 36.5) (end 80 37.75) (width 0.25) (layer "F.Cu") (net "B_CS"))
 (segment (start 79.25 56) (end 81 57.75) (width 0.25) (layer "F.Cu") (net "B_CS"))
 (segment (start 81 57.75) (end 81 58) (width 0.25) (layer "F.Cu") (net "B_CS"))
 (via (at 81 58) (size 0.7) (drill 0.3) (layers "F.Cu" "B.Cu") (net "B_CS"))
 (segment (start 73 83.3) (end 81 83.3) (width 0.25) (layer "B.Cu") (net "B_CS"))
 (segment (start 81 83.3) (end 81 58) (width 0.25) (layer "B.Cu") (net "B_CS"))
 (segment (start 88.5 39) (end 85.25 42.25) (width 0.25) (layer "F.Cu") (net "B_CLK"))
 (segment (start 89.25 39) (end 88.5 39) (width 0.25) (layer "F.Cu") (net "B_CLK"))
 (segment (start 89.5875 38.635) (end 89.5 38.75) (width 0.25) (layer "F.Cu") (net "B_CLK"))
 (segment (start 89.5 38.75) (end 89.25 39) (width 0.25) (layer "F.Cu") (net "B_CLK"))
 (via (at 85.25 42.25) (size 0.7) (drill 0.3) (layers "F.Cu" "B.Cu") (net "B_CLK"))
 (segment (start 85.25 42.25) (end 82.5 45) (width 0.25) (layer "B.Cu") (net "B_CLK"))
 (segment (start 73 89.3) (end 82.5 89.3) (width 0.25) (layer "B.Cu") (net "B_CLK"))
 (segment (start 82.5 89.3) (end 82.5 58) (width 0.25) (layer "B.Cu") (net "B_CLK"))
 (segment (start 82.5 45) (end 82.5 58) (width 0.25) (layer "B.Cu") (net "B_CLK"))
 (segment (start 84 53.25) (end 84 58) (width 0.25) (layer "F.Cu") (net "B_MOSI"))
 (segment (start 89.25 48) (end 84 53.25) (width 0.25) (layer "F.Cu") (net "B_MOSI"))
 (segment (start 89.25 40.25) (end 89.25 48) (width 0.25) (layer "F.Cu") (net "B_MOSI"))
 (segment (start 89.5875 39.905) (end 89.5 40) (width 0.25) (layer "F.Cu") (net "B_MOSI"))
 (segment (start 89.5 40) (end 89.25 40.25) (width 0.25) (layer "F.Cu") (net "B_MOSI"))
 (via (at 84 58) (size 0.7) (drill 0.3) (layers "F.Cu" "B.Cu") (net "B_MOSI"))
 (segment (start 73 95.3) (end 84 95.3) (width 0.25) (layer "B.Cu") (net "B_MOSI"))
 (segment (start 84 95.3) (end 84 58) (width 0.25) (layer "B.Cu") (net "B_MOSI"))
 (segment (start 83.5 37.75) (end 83.75 38) (width 0.25) (layer "F.Cu") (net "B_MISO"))
 (segment (start 83.75 38) (end 83.75 44.25) (width 0.25) (layer "F.Cu") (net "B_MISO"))
 (segment (start 83 37.75) (end 83.5 37.75) (width 0.25) (layer "F.Cu") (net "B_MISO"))
 (segment (start 83.75 44.25) (end 85.5 46) (width 0.25) (layer "F.Cu") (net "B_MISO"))
 (segment (start 85.5 46) (end 85.5 46.25) (width 0.25) (layer "F.Cu") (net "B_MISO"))
 (segment (start 82.4125 37.365) (end 82.5 37.25) (width 0.25) (layer "F.Cu") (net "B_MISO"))
 (segment (start 82.5 37.25) (end 83 37.75) (width 0.25) (layer "F.Cu") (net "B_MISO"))
 (via (at 85.5 46.25) (size 0.7) (drill 0.3) (layers "F.Cu" "B.Cu") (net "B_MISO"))
 (segment (start 73 101.3) (end 85.5 101.3) (width 0.25) (layer "B.Cu") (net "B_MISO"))
 (segment (start 85.5 101.3) (end 85.5 58) (width 0.25) (layer "B.Cu") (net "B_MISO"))
 (segment (start 85.5 46.25) (end 85.5 58) (width 0.25) (layer "B.Cu") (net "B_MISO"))
 (segment (start 87 48.25) (end 87 48) (width 0.25) (layer "F.Cu") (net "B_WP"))
 (segment (start 87 48) (end 86.9125 48) (width 0.25) (layer "F.Cu") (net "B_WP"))
 (segment (start 81 39.25) (end 81 40.5) (width 0.25) (layer "F.Cu") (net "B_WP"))
 (segment (start 84 49) (end 84.25 49.25) (width 0.25) (layer "F.Cu") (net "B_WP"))
 (segment (start 82.4125 38.635) (end 82.5 38.75) (width 0.25) (layer "F.Cu") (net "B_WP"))
 (segment (start 81.25 39) (end 81 39.25) (width 0.25) (layer "F.Cu") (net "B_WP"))
 (segment (start 81.25 45.25) (end 84 48) (width 0.25) (layer "F.Cu") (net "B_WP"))
 (segment (start 84 48) (end 84 49) (width 0.25) (layer "F.Cu") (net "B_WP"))
 (segment (start 86 49.25) (end 87 48.25) (width 0.25) (layer "F.Cu") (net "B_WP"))
 (segment (start 82.5 38.75) (end 82.25 39) (width 0.25) (layer "F.Cu") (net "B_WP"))
 (segment (start 81.25 40.75) (end 81.25 45.25) (width 0.25) (layer "F.Cu") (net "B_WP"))
 (segment (start 84.25 49.25) (end 86 49.25) (width 0.25) (layer "F.Cu") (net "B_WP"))
 (segment (start 82.25 39) (end 81.25 39) (width 0.25) (layer "F.Cu") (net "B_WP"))
 (segment (start 81 40.5) (end 81.25 40.75) (width 0.25) (layer "F.Cu") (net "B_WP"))
 (segment (start 89.5875 37.365) (end 89.5 37.25) (width 0.25) (layer "F.Cu") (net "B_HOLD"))
 (segment (start 95 48) (end 94.9125 48) (width 0.25) (layer "F.Cu") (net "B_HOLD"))
 (segment (start 90 37.75) (end 90.75 37.75) (width 0.25) (layer "F.Cu") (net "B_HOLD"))
 (segment (start 89.5 37.25) (end 90 37.75) (width 0.25) (layer "F.Cu") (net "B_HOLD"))
 (segment (start 90.75 37.75) (end 94 41) (width 0.25) (layer "F.Cu") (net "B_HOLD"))
 (segment (start 94 42.75) (end 95 43.75) (width 0.25) (layer "F.Cu") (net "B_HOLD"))
 (segment (start 95 43.75) (end 95 48) (width 0.25) (layer "F.Cu") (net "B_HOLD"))
 (segment (start 94 41) (end 94 42.75) (width 0.25) (layer "F.Cu") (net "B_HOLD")))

